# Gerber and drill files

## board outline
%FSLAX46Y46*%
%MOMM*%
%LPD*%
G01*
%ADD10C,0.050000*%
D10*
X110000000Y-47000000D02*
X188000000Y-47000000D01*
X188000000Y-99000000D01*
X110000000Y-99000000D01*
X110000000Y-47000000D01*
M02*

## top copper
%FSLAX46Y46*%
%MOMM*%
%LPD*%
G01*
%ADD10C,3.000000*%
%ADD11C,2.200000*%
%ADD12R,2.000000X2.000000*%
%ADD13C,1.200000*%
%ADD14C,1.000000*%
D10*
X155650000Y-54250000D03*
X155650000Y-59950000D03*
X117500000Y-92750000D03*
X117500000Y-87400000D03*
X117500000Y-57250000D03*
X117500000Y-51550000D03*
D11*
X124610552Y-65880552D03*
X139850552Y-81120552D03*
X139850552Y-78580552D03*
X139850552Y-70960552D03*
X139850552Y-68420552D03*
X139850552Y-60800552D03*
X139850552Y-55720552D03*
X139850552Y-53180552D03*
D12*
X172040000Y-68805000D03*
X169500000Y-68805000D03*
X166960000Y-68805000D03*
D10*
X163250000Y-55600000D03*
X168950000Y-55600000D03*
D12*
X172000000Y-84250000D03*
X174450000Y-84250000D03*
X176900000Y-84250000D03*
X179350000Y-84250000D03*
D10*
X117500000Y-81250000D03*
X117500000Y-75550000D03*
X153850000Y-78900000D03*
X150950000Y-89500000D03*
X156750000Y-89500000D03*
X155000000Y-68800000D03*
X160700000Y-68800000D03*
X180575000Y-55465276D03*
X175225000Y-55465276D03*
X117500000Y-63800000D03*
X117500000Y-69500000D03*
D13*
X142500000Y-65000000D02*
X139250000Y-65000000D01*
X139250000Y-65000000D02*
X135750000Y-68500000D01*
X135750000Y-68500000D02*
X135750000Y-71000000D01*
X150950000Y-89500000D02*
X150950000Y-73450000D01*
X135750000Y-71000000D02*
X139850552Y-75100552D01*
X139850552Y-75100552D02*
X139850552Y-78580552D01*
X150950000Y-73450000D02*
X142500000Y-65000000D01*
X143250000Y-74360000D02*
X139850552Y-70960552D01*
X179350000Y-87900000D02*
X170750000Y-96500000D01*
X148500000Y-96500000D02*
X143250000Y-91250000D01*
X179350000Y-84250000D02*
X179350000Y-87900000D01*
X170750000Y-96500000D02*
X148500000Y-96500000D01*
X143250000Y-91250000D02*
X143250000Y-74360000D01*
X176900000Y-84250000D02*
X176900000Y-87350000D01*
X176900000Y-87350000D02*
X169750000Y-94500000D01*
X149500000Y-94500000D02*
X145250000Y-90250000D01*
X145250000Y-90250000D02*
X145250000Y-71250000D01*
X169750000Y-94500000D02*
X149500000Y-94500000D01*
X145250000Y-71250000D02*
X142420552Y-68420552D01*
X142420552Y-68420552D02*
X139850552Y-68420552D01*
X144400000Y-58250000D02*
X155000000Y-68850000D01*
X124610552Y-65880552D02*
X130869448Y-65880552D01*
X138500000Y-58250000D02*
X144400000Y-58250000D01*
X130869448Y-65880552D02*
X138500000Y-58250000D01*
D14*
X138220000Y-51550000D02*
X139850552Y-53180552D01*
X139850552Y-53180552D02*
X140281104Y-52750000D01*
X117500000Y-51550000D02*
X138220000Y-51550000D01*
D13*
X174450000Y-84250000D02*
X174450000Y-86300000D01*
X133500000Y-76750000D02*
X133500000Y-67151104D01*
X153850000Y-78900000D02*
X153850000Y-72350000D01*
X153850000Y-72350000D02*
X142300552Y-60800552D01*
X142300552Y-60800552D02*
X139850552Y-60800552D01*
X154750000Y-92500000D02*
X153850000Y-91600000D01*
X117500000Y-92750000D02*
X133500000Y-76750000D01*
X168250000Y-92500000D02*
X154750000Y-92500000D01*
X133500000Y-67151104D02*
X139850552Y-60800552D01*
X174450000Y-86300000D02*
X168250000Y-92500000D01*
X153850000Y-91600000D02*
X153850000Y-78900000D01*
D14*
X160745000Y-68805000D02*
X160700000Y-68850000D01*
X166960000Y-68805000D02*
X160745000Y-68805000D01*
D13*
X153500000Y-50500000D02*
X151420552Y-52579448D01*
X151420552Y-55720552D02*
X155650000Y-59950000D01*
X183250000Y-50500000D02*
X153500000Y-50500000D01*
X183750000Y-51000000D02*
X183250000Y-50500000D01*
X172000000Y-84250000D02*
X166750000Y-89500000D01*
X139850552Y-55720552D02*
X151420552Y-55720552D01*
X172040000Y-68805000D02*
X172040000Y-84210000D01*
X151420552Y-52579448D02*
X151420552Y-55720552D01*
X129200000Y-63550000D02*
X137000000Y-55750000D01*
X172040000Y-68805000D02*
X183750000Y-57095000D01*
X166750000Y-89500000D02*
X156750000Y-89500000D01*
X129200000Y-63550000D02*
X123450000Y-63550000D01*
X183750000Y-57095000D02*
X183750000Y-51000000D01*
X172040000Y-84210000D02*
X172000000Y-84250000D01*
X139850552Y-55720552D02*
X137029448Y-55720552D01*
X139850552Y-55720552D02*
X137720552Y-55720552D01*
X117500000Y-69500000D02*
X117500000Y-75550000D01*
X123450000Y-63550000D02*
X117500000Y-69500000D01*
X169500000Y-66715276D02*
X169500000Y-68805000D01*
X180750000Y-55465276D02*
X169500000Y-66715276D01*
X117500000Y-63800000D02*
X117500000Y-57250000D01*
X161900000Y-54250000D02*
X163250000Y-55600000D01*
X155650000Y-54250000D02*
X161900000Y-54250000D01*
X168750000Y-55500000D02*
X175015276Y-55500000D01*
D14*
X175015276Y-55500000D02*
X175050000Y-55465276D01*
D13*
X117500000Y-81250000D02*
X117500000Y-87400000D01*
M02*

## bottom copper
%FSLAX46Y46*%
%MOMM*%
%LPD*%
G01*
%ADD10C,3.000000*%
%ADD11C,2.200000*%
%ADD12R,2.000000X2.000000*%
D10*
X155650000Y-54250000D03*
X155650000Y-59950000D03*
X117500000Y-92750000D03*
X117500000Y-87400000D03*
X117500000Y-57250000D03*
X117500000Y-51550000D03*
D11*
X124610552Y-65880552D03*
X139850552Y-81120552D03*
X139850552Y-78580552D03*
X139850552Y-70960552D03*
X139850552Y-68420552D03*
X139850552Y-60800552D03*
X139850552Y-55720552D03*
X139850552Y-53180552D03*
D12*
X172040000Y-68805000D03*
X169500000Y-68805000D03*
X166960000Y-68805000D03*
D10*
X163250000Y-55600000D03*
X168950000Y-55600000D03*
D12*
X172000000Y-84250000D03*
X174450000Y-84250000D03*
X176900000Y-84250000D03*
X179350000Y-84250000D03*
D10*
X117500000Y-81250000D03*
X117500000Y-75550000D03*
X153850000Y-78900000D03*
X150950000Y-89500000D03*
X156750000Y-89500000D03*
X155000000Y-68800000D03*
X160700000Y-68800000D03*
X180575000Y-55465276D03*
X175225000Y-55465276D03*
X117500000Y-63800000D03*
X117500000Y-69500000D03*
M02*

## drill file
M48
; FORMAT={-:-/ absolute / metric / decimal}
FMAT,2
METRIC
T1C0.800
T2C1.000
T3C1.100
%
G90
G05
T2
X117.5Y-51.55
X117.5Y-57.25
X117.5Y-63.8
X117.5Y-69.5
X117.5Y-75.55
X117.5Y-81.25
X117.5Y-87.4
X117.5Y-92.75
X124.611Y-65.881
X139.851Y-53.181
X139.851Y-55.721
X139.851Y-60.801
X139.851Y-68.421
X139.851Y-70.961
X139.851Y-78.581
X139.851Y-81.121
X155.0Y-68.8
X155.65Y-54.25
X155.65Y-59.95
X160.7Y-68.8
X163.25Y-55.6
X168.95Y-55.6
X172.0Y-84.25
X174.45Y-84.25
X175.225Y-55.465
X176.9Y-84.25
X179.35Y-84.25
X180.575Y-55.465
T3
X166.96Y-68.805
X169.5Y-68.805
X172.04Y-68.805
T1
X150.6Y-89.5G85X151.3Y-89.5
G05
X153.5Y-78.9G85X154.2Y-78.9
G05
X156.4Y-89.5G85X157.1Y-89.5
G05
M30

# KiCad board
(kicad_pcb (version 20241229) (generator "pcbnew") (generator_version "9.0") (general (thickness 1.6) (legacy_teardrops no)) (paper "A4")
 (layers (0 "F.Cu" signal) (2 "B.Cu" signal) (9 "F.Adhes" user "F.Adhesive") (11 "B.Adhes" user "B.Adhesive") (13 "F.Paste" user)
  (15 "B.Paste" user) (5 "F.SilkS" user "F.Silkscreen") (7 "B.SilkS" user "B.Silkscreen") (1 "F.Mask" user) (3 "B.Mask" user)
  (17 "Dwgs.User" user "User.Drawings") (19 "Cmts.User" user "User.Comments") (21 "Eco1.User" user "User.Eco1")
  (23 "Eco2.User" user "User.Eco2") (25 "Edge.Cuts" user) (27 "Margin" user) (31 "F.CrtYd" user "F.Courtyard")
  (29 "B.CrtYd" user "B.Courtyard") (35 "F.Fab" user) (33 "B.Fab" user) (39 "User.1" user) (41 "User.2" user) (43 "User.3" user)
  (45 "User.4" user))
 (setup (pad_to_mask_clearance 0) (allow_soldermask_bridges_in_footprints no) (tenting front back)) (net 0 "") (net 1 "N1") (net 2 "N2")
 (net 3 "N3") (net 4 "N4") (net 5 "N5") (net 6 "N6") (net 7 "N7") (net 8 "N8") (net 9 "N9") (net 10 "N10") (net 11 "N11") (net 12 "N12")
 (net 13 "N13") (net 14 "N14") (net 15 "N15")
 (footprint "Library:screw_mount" (layer "F.Cu") (at 159.45 51.75 -90)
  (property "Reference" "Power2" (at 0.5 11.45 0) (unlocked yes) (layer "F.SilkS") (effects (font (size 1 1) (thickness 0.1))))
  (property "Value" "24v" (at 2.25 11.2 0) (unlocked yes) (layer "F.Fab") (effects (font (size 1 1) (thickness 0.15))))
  (pad "1" thru_hole circle (at 2.5 3.8 270) (size 3 3) (drill 1) (layers "*.Cu" "*.Mask") (remove_unused_layers no) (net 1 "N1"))
  (pad "2" thru_hole circle (at 8.2 3.8 270) (size 3 3) (drill 1) (layers "*.Cu" "*.Mask") (remove_unused_layers no) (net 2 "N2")))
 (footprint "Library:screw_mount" (layer "F.Cu") (at 113.7 95.425 90)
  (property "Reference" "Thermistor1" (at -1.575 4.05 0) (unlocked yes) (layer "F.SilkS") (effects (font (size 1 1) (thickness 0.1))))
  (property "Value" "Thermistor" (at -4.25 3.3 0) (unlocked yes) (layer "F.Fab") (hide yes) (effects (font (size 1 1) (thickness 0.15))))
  (pad "1" thru_hole circle (at 2.675 3.8 90) (size 3 3) (drill 1) (layers "*.Cu" "*.Mask") (remove_unused_layers no) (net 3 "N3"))
  (pad "2" thru_hole circle (at 8.025 3.8 90) (size 3 3) (drill 1) (layers "*.Cu" "*.Mask") (remove_unused_layers no) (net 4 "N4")))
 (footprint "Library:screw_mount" (layer "F.Cu") (at 113.7 59.75 90)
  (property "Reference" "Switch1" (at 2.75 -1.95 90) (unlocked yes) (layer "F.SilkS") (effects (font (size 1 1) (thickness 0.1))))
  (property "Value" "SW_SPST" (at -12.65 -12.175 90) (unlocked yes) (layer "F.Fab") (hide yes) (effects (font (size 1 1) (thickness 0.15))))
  (pad "1" thru_hole circle (at 2.5 3.8 90) (size 3 3) (drill 1) (layers "*.Cu" "*.Mask") (remove_unused_layers no) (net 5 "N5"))
  (pad "2" thru_hole circle (at 8.2 3.8 90) (size 3 3) (drill 1) (layers "*.Cu" "*.Mask") (remove_unused_layers no) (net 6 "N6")))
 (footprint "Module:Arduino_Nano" (layer "F.Cu") (at 124.610552 53.180552)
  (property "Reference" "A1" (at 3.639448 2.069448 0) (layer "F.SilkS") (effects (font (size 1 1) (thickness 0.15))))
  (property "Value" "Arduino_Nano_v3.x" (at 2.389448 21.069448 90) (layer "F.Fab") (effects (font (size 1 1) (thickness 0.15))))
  (pad "6" thru_hole circle (at 0 12.7) (size 2.2 2.2) (drill 1) (layers "*.Cu" "*.Mask") (remove_unused_layers no) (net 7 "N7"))
  (pad "19" thru_hole circle (at 15.24 27.94) (size 2.2 2.2) (drill 1) (layers "*.Cu" "*.Mask") (remove_unused_layers no) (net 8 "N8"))
  (pad "20" thru_hole circle (at 15.24 25.4) (size 2.2 2.2) (drill 1) (layers "*.Cu" "*.Mask") (remove_unused_layers no) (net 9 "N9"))
  (pad "23" thru_hole circle (at 15.24 17.78) (size 2.2 2.2) (drill 1) (layers "*.Cu" "*.Mask") (remove_unused_layers no) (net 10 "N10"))
  (pad "24" thru_hole circle (at 15.24 15.24) (size 2.2 2.2) (drill 1) (layers "*.Cu" "*.Mask") (remove_unused_layers no) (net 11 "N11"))
  (pad "27" thru_hole circle (at 15.24 7.62) (size 2.2 2.2) (drill 1) (layers "*.Cu" "*.Mask") (remove_unused_layers no) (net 3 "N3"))
  (pad "29" thru_hole circle (at 15.24 2.54) (size 2.2 2.2) (drill 1) (layers "*.Cu" "*.Mask") (remove_unused_layers no) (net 2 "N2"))
  (pad "30" thru_hole circle (at 15.24 0) (size 2.2 2.2) (drill 1) (layers "*.Cu" "*.Mask") (remove_unused_layers no) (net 6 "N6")))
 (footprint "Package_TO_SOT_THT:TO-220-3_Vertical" (layer "F.Cu") (at 172.04 68.805 180)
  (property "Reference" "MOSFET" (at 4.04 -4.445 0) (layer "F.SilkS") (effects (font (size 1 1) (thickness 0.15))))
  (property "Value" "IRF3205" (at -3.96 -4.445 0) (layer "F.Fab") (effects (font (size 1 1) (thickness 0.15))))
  (pad "1" thru_hole rect (at 0 0 180) (size 2 2) (drill 1.1) (layers "*.Cu" "*.Mask") (remove_unused_layers no) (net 2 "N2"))
  (pad "2" thru_hole rect (at 2.54 0 180) (size 2 2) (drill 1.1) (layers "*.Cu" "*.Mask") (remove_unused_layers no) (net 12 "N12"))
  (pad "3" thru_hole rect (at 5.08 0 180) (size 2 2) (drill 1.1) (layers "*.Cu" "*.Mask") (remove_unused_layers no) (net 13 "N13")))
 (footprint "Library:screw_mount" (layer "F.Cu") (at 160.75 51.8)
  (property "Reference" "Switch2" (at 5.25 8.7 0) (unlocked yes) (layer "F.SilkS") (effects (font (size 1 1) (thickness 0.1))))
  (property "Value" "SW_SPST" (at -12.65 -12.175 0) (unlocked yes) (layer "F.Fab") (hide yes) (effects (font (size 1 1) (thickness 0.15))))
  (pad "1" thru_hole circle (at 2.5 3.8) (size 3 3) (drill 1) (layers "*.Cu" "*.Mask") (remove_unused_layers no) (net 1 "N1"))
  (pad "2" thru_hole circle (at 8.2 3.8) (size 3 3) (drill 1) (layers "*.Cu" "*.Mask") (remove_unused_layers no) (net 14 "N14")))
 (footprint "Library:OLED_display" (layer "F.Cu") (at 170.775 85.45 90)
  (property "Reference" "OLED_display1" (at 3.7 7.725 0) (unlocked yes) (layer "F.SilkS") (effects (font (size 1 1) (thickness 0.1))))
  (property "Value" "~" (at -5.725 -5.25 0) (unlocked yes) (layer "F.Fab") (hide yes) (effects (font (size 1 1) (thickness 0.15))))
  (pad "1" thru_hole rect (at 1.2 1.225 90) (size 2 2) (drill 1) (layers "*.Cu" "*.Mask") (remove_unused_layers no) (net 2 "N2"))
  (pad "2" thru_hole rect (at 1.2 3.675 90) (size 2 2) (drill 1) (layers "*.Cu" "*.Mask") (remove_unused_layers no) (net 3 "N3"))
  (pad "3" thru_hole rect (at 1.2 6.125 90) (size 2 2) (drill 1) (layers "*.Cu" "*.Mask") (remove_unused_layers no) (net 11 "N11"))
  (pad "4" thru_hole rect (at 1.2 8.575 90) (size 2 2) (drill 1) (layers "*.Cu" "*.Mask") (remove_unused_layers no) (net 10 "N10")))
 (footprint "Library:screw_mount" (layer "F.Cu") (at 113.7 83.75 90)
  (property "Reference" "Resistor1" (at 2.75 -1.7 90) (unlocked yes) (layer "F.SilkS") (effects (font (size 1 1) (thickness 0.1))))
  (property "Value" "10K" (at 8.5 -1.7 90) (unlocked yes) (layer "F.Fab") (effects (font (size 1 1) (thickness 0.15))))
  (pad "1" thru_hole circle (at 2.5 3.8 90) (size 3 3) (drill 1) (layers "*.Cu" "*.Mask") (remove_unused_layers no) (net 4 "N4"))
  (pad "2" thru_hole circle (at 8.2 3.8 90) (size 3 3) (drill 1) (layers "*.Cu" "*.Mask") (remove_unused_layers no) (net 2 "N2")))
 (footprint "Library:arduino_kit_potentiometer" (layer "F.Cu") (at 148.95 78.9)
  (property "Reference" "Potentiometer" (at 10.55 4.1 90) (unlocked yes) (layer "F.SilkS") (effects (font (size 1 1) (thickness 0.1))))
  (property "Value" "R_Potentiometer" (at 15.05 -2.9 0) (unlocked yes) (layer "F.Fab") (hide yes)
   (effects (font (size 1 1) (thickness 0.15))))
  (pad "1" thru_hole circle (at 4.9 0) (size 3 3) (drill oval 1.5 0.8) (layers "*.Cu" "*.Mask") (remove_unused_layers no) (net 3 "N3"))
  (pad "2" thru_hole circle (at 2 10.6) (size 3 3) (drill oval 1.5 0.8) (layers "*.Cu" "*.Mask") (remove_unused_layers no) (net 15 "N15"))
  (pad "3" thru_hole circle (at 7.8 10.6) (size 3 3) (drill oval 1.5 0.8) (layers "*.Cu" "*.Mask") (remove_unused_layers no) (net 2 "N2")))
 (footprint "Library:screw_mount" (layer "F.Cu") (at 152.5 65)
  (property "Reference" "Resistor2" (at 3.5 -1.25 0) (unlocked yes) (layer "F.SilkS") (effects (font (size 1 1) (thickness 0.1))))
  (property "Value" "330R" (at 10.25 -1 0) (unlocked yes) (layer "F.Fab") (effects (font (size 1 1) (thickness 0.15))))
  (pad "1" thru_hole circle (at 2.5 3.8) (size 3 3) (drill 1) (layers "*.Cu" "*.Mask") (remove_unused_layers no) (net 7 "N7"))
  (pad "2" thru_hole circle (at 8.2 3.8) (size 3 3) (drill 1) (layers "*.Cu" "*.Mask") (remove_unused_layers no) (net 13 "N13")))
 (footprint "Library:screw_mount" (layer "F.Cu") (at 183.25 59.265276 180)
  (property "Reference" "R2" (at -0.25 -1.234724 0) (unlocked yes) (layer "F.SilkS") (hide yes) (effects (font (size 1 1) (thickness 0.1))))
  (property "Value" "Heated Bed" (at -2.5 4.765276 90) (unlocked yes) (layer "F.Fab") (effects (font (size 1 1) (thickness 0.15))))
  (pad "1" thru_hole circle (at 2.675 3.8 180) (size 3 3) (drill 1) (layers "*.Cu" "*.Mask") (remove_unused_layers no) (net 12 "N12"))
  (pad "2" thru_hole circle (at 8.025 3.8 180) (size 3 3) (drill 1) (layers "*.Cu" "*.Mask") (remove_unused_layers no) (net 14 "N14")))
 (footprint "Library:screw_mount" (layer "F.Cu") (at 121.3 61.3 -90)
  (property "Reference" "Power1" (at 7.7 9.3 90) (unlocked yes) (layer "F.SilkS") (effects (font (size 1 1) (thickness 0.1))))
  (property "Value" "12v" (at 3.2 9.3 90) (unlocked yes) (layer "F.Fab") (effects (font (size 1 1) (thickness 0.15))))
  (pad "1" thru_hole circle (at 2.5 3.8 270) (size 3 3) (drill 1) (layers "*.Cu" "*.Mask") (remove_unused_layers no) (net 5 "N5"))
  (pad "2" thru_hole circle (at 8.2 3.8 270) (size 3 3) (drill 1) (layers "*.Cu" "*.Mask") (remove_unused_layers no) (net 2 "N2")))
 (gr_rect (start 110 47) (end 188 99) (stroke (width 0.05) (type default)) (fill no) (layer "Edge.Cuts"))
 (segment (start 142.5 65) (end 139.25 65) (width 1.2) (layer "F.Cu") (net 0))
 (segment (start 139.25 65) (end 135.75 68.5) (width 1.2) (layer "F.Cu") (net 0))
 (segment (start 135.75 68.5) (end 135.75 71) (width 1.2) (layer "F.Cu") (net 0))
 (segment (start 150.95 89.5) (end 150.95 73.45) (width 1.2) (layer "F.Cu") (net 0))
 (segment (start 135.75 71) (end 139.850552 75.100552) (width 1.2) (layer "F.Cu") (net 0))
 (segment (start 139.850552 75.100552) (end 139.850552 78.580552) (width 1.2) (layer "F.Cu") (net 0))
 (segment (start 150.95 73.45) (end 142.5 65) (width 1.2) (layer "F.Cu") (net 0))
 (segment (start 143.25 74.36) (end 139.850552 70.960552) (width 1.2) (layer "F.Cu") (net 10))
 (segment (start 179.35 87.9) (end 170.75 96.5) (width 1.2) (layer "F.Cu") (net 10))
 (segment (start 148.5 96.5) (end 143.25 91.25) (width 1.2) (layer "F.Cu") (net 10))
 (segment (start 179.35 84.25) (end 179.35 87.9) (width 1.2) (layer "F.Cu") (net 10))
 (segment (start 170.75 96.5) (end 148.5 96.5) (width 1.2) (layer "F.Cu") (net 10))
 (segment (start 143.25 91.25) (end 143.25 74.36) (width 1.2) (layer "F.Cu") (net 10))
 (segment (start 176.9 84.25) (end 176.9 87.35) (width 1.2) (layer "F.Cu") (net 11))
 (segment (start 176.9 87.35) (end 169.75 94.5) (width 1.2) (layer "F.Cu") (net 11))
 (segment (start 149.5 94.5) (end 145.25 90.25) (width 1.2) (layer "F.Cu") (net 11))
 (segment (start 145.25 90.25) (end 145.25 71.25) (width 1.2) (layer "F.Cu") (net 11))
 (segment (start 169.75 94.5) (end 149.5 94.5) (width 1.2) (layer "F.Cu") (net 11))
 (segment (start 145.25 71.25) (end 142.420552 68.420552) (width 1.2) (layer "F.Cu") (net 11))
 (segment (start 142.420552 68.420552) (end 139.850552 68.420552) (width 1.2) (layer "F.Cu") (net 11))
 (segment (start 144.4 58.25) (end 155 68.85) (width 1.2) (layer "F.Cu") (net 7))
 (segment (start 124.610552 65.880552) (end 130.869448 65.880552) (width 1.2) (layer "F.Cu") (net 7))
 (segment (start 138.5 58.25) (end 144.4 58.25) (width 1.2) (layer "F.Cu") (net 7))
 (segment (start 130.869448 65.880552) (end 138.5 58.25) (width 1.2) (layer "F.Cu") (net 7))
 (segment (start 138.22 51.55) (end 139.850552 53.180552) (width 1) (layer "F.Cu") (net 6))
 (segment (start 139.850552 53.180552) (end 140.281104 52.75) (width 1) (layer "F.Cu") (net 6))
 (segment (start 117.5 51.55) (end 138.22 51.55) (width 1) (layer "F.Cu") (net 6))
 (segment (start 174.45 84.25) (end 174.45 86.3) (width 1.2) (layer "F.Cu") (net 3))
 (segment (start 133.5 76.75) (end 133.5 67.151104) (width 1.2) (layer "F.Cu") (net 3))
 (segment (start 153.85 78.9) (end 153.85 72.35) (width 1.2) (layer "F.Cu") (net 3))
 (segment (start 153.85 72.35) (end 142.300552 60.800552) (width 1.2) (layer "F.Cu") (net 3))
 (segment (start 142.300552 60.800552) (end 139.850552 60.800552) (width 1.2) (layer "F.Cu") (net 3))
 (segment (start 154.75 92.5) (end 153.85 91.6) (width 1.2) (layer "F.Cu") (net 3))
 (segment (start 117.5 92.75) (end 133.5 76.75) (width 1.2) (layer "F.Cu") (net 3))
 (segment (start 168.25 92.5) (end 154.75 92.5) (width 1.2) (layer "F.Cu") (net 3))
 (segment (start 133.5 67.151104) (end 139.850552 60.800552) (width 1.2) (layer "F.Cu") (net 3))
 (segment (start 174.45 86.3) (end 168.25 92.5) (width 1.2) (layer "F.Cu") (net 3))
 (segment (start 153.85 91.6) (end 153.85 78.9) (width 1.2) (layer "F.Cu") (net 3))
 (segment (start 160.745 68.805) (end 160.7 68.85) (width 1) (layer "F.Cu") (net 13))
 (segment (start 166.96 68.805) (end 160.745 68.805) (width 1) (layer "F.Cu") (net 13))
 (segment (start 153.5 50.5) (end 151.420552 52.579448) (width 1.2) (layer "F.Cu") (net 2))
 (segment (start 151.420552 55.720552) (end 155.65 59.95) (width 1.2) (layer "F.Cu") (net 2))
 (segment (start 183.25 50.5) (end 153.5 50.5) (width 1.2) (layer "F.Cu") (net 2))
 (segment (start 183.75 51) (end 183.25 50.5) (width 1.2) (layer "F.Cu") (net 2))
 (segment (start 172 84.25) (end 166.75 89.5) (width 1.2) (layer "F.Cu") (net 2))
 (segment (start 139.850552 55.720552) (end 151.420552 55.720552) (width 1.2) (layer "F.Cu") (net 2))
 (segment (start 172.04 68.805) (end 172.04 84.21) (width 1.2) (layer "F.Cu") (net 2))
 (segment (start 151.420552 52.579448) (end 151.420552 55.720552) (width 1.2) (layer "F.Cu") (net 2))
 (segment (start 129.2 63.55) (end 137 55.75) (width 1.2) (layer "F.Cu") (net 2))
 (segment (start 172.04 68.805) (end 183.75 57.095) (width 1.2) (layer "F.Cu") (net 2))
 (segment (start 166.75 89.5) (end 156.75 89.5) (width 1.2) (layer "F.Cu") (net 2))
 (segment (start 129.2 63.55) (end 123.45 63.55) (width 1.2) (layer "F.Cu") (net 2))
 (segment (start 183.75 57.095) (end 183.75 51) (width 1.2) (layer "F.Cu") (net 2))
 (segment (start 172.04 84.21) (end 172 84.25) (width 1.2) (layer "F.Cu") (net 2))
 (segment (start 139.850552 55.720552) (end 137.029448 55.720552) (width 1.2) (layer "F.Cu") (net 2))
 (segment (start 139.850552 55.720552) (end 137.720552 55.720552) (width 1.2) (layer "F.Cu") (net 2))
 (segment (start 117.5 69.5) (end 117.5 75.55) (width 1.2) (layer "F.Cu") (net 2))
 (segment (start 123.45 63.55) (end 117.5 69.5) (width 1.2) (layer "F.Cu") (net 2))
 (segment (start 169.5 66.715276) (end 169.5 68.805) (width 1.2) (layer "F.Cu") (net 12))
 (segment (start 180.75 55.465276) (end 169.5 66.715276) (width 1.2) (layer "F.Cu") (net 12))
 (segment (start 117.5 63.8) (end 117.5 57.25) (width 1.2) (layer "F.Cu") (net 5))
 (segment (start 161.9 54.25) (end 163.25 55.6) (width 1.2) (layer "F.Cu") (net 1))
 (segment (start 155.65 54.25) (end 161.9 54.25) (width 1.2) (layer "F.Cu") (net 1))
 (segment (start 168.75 55.5) (end 175.015276 55.5) (width 1.2) (layer "F.Cu") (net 14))
 (segment (start 175.015276 55.5) (end 175.05 55.465276) (width 1) (layer "F.Cu") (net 14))
 (segment (start 117.5 81.25) (end 117.5 87.4) (width 1.2) (layer "F.Cu") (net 4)))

